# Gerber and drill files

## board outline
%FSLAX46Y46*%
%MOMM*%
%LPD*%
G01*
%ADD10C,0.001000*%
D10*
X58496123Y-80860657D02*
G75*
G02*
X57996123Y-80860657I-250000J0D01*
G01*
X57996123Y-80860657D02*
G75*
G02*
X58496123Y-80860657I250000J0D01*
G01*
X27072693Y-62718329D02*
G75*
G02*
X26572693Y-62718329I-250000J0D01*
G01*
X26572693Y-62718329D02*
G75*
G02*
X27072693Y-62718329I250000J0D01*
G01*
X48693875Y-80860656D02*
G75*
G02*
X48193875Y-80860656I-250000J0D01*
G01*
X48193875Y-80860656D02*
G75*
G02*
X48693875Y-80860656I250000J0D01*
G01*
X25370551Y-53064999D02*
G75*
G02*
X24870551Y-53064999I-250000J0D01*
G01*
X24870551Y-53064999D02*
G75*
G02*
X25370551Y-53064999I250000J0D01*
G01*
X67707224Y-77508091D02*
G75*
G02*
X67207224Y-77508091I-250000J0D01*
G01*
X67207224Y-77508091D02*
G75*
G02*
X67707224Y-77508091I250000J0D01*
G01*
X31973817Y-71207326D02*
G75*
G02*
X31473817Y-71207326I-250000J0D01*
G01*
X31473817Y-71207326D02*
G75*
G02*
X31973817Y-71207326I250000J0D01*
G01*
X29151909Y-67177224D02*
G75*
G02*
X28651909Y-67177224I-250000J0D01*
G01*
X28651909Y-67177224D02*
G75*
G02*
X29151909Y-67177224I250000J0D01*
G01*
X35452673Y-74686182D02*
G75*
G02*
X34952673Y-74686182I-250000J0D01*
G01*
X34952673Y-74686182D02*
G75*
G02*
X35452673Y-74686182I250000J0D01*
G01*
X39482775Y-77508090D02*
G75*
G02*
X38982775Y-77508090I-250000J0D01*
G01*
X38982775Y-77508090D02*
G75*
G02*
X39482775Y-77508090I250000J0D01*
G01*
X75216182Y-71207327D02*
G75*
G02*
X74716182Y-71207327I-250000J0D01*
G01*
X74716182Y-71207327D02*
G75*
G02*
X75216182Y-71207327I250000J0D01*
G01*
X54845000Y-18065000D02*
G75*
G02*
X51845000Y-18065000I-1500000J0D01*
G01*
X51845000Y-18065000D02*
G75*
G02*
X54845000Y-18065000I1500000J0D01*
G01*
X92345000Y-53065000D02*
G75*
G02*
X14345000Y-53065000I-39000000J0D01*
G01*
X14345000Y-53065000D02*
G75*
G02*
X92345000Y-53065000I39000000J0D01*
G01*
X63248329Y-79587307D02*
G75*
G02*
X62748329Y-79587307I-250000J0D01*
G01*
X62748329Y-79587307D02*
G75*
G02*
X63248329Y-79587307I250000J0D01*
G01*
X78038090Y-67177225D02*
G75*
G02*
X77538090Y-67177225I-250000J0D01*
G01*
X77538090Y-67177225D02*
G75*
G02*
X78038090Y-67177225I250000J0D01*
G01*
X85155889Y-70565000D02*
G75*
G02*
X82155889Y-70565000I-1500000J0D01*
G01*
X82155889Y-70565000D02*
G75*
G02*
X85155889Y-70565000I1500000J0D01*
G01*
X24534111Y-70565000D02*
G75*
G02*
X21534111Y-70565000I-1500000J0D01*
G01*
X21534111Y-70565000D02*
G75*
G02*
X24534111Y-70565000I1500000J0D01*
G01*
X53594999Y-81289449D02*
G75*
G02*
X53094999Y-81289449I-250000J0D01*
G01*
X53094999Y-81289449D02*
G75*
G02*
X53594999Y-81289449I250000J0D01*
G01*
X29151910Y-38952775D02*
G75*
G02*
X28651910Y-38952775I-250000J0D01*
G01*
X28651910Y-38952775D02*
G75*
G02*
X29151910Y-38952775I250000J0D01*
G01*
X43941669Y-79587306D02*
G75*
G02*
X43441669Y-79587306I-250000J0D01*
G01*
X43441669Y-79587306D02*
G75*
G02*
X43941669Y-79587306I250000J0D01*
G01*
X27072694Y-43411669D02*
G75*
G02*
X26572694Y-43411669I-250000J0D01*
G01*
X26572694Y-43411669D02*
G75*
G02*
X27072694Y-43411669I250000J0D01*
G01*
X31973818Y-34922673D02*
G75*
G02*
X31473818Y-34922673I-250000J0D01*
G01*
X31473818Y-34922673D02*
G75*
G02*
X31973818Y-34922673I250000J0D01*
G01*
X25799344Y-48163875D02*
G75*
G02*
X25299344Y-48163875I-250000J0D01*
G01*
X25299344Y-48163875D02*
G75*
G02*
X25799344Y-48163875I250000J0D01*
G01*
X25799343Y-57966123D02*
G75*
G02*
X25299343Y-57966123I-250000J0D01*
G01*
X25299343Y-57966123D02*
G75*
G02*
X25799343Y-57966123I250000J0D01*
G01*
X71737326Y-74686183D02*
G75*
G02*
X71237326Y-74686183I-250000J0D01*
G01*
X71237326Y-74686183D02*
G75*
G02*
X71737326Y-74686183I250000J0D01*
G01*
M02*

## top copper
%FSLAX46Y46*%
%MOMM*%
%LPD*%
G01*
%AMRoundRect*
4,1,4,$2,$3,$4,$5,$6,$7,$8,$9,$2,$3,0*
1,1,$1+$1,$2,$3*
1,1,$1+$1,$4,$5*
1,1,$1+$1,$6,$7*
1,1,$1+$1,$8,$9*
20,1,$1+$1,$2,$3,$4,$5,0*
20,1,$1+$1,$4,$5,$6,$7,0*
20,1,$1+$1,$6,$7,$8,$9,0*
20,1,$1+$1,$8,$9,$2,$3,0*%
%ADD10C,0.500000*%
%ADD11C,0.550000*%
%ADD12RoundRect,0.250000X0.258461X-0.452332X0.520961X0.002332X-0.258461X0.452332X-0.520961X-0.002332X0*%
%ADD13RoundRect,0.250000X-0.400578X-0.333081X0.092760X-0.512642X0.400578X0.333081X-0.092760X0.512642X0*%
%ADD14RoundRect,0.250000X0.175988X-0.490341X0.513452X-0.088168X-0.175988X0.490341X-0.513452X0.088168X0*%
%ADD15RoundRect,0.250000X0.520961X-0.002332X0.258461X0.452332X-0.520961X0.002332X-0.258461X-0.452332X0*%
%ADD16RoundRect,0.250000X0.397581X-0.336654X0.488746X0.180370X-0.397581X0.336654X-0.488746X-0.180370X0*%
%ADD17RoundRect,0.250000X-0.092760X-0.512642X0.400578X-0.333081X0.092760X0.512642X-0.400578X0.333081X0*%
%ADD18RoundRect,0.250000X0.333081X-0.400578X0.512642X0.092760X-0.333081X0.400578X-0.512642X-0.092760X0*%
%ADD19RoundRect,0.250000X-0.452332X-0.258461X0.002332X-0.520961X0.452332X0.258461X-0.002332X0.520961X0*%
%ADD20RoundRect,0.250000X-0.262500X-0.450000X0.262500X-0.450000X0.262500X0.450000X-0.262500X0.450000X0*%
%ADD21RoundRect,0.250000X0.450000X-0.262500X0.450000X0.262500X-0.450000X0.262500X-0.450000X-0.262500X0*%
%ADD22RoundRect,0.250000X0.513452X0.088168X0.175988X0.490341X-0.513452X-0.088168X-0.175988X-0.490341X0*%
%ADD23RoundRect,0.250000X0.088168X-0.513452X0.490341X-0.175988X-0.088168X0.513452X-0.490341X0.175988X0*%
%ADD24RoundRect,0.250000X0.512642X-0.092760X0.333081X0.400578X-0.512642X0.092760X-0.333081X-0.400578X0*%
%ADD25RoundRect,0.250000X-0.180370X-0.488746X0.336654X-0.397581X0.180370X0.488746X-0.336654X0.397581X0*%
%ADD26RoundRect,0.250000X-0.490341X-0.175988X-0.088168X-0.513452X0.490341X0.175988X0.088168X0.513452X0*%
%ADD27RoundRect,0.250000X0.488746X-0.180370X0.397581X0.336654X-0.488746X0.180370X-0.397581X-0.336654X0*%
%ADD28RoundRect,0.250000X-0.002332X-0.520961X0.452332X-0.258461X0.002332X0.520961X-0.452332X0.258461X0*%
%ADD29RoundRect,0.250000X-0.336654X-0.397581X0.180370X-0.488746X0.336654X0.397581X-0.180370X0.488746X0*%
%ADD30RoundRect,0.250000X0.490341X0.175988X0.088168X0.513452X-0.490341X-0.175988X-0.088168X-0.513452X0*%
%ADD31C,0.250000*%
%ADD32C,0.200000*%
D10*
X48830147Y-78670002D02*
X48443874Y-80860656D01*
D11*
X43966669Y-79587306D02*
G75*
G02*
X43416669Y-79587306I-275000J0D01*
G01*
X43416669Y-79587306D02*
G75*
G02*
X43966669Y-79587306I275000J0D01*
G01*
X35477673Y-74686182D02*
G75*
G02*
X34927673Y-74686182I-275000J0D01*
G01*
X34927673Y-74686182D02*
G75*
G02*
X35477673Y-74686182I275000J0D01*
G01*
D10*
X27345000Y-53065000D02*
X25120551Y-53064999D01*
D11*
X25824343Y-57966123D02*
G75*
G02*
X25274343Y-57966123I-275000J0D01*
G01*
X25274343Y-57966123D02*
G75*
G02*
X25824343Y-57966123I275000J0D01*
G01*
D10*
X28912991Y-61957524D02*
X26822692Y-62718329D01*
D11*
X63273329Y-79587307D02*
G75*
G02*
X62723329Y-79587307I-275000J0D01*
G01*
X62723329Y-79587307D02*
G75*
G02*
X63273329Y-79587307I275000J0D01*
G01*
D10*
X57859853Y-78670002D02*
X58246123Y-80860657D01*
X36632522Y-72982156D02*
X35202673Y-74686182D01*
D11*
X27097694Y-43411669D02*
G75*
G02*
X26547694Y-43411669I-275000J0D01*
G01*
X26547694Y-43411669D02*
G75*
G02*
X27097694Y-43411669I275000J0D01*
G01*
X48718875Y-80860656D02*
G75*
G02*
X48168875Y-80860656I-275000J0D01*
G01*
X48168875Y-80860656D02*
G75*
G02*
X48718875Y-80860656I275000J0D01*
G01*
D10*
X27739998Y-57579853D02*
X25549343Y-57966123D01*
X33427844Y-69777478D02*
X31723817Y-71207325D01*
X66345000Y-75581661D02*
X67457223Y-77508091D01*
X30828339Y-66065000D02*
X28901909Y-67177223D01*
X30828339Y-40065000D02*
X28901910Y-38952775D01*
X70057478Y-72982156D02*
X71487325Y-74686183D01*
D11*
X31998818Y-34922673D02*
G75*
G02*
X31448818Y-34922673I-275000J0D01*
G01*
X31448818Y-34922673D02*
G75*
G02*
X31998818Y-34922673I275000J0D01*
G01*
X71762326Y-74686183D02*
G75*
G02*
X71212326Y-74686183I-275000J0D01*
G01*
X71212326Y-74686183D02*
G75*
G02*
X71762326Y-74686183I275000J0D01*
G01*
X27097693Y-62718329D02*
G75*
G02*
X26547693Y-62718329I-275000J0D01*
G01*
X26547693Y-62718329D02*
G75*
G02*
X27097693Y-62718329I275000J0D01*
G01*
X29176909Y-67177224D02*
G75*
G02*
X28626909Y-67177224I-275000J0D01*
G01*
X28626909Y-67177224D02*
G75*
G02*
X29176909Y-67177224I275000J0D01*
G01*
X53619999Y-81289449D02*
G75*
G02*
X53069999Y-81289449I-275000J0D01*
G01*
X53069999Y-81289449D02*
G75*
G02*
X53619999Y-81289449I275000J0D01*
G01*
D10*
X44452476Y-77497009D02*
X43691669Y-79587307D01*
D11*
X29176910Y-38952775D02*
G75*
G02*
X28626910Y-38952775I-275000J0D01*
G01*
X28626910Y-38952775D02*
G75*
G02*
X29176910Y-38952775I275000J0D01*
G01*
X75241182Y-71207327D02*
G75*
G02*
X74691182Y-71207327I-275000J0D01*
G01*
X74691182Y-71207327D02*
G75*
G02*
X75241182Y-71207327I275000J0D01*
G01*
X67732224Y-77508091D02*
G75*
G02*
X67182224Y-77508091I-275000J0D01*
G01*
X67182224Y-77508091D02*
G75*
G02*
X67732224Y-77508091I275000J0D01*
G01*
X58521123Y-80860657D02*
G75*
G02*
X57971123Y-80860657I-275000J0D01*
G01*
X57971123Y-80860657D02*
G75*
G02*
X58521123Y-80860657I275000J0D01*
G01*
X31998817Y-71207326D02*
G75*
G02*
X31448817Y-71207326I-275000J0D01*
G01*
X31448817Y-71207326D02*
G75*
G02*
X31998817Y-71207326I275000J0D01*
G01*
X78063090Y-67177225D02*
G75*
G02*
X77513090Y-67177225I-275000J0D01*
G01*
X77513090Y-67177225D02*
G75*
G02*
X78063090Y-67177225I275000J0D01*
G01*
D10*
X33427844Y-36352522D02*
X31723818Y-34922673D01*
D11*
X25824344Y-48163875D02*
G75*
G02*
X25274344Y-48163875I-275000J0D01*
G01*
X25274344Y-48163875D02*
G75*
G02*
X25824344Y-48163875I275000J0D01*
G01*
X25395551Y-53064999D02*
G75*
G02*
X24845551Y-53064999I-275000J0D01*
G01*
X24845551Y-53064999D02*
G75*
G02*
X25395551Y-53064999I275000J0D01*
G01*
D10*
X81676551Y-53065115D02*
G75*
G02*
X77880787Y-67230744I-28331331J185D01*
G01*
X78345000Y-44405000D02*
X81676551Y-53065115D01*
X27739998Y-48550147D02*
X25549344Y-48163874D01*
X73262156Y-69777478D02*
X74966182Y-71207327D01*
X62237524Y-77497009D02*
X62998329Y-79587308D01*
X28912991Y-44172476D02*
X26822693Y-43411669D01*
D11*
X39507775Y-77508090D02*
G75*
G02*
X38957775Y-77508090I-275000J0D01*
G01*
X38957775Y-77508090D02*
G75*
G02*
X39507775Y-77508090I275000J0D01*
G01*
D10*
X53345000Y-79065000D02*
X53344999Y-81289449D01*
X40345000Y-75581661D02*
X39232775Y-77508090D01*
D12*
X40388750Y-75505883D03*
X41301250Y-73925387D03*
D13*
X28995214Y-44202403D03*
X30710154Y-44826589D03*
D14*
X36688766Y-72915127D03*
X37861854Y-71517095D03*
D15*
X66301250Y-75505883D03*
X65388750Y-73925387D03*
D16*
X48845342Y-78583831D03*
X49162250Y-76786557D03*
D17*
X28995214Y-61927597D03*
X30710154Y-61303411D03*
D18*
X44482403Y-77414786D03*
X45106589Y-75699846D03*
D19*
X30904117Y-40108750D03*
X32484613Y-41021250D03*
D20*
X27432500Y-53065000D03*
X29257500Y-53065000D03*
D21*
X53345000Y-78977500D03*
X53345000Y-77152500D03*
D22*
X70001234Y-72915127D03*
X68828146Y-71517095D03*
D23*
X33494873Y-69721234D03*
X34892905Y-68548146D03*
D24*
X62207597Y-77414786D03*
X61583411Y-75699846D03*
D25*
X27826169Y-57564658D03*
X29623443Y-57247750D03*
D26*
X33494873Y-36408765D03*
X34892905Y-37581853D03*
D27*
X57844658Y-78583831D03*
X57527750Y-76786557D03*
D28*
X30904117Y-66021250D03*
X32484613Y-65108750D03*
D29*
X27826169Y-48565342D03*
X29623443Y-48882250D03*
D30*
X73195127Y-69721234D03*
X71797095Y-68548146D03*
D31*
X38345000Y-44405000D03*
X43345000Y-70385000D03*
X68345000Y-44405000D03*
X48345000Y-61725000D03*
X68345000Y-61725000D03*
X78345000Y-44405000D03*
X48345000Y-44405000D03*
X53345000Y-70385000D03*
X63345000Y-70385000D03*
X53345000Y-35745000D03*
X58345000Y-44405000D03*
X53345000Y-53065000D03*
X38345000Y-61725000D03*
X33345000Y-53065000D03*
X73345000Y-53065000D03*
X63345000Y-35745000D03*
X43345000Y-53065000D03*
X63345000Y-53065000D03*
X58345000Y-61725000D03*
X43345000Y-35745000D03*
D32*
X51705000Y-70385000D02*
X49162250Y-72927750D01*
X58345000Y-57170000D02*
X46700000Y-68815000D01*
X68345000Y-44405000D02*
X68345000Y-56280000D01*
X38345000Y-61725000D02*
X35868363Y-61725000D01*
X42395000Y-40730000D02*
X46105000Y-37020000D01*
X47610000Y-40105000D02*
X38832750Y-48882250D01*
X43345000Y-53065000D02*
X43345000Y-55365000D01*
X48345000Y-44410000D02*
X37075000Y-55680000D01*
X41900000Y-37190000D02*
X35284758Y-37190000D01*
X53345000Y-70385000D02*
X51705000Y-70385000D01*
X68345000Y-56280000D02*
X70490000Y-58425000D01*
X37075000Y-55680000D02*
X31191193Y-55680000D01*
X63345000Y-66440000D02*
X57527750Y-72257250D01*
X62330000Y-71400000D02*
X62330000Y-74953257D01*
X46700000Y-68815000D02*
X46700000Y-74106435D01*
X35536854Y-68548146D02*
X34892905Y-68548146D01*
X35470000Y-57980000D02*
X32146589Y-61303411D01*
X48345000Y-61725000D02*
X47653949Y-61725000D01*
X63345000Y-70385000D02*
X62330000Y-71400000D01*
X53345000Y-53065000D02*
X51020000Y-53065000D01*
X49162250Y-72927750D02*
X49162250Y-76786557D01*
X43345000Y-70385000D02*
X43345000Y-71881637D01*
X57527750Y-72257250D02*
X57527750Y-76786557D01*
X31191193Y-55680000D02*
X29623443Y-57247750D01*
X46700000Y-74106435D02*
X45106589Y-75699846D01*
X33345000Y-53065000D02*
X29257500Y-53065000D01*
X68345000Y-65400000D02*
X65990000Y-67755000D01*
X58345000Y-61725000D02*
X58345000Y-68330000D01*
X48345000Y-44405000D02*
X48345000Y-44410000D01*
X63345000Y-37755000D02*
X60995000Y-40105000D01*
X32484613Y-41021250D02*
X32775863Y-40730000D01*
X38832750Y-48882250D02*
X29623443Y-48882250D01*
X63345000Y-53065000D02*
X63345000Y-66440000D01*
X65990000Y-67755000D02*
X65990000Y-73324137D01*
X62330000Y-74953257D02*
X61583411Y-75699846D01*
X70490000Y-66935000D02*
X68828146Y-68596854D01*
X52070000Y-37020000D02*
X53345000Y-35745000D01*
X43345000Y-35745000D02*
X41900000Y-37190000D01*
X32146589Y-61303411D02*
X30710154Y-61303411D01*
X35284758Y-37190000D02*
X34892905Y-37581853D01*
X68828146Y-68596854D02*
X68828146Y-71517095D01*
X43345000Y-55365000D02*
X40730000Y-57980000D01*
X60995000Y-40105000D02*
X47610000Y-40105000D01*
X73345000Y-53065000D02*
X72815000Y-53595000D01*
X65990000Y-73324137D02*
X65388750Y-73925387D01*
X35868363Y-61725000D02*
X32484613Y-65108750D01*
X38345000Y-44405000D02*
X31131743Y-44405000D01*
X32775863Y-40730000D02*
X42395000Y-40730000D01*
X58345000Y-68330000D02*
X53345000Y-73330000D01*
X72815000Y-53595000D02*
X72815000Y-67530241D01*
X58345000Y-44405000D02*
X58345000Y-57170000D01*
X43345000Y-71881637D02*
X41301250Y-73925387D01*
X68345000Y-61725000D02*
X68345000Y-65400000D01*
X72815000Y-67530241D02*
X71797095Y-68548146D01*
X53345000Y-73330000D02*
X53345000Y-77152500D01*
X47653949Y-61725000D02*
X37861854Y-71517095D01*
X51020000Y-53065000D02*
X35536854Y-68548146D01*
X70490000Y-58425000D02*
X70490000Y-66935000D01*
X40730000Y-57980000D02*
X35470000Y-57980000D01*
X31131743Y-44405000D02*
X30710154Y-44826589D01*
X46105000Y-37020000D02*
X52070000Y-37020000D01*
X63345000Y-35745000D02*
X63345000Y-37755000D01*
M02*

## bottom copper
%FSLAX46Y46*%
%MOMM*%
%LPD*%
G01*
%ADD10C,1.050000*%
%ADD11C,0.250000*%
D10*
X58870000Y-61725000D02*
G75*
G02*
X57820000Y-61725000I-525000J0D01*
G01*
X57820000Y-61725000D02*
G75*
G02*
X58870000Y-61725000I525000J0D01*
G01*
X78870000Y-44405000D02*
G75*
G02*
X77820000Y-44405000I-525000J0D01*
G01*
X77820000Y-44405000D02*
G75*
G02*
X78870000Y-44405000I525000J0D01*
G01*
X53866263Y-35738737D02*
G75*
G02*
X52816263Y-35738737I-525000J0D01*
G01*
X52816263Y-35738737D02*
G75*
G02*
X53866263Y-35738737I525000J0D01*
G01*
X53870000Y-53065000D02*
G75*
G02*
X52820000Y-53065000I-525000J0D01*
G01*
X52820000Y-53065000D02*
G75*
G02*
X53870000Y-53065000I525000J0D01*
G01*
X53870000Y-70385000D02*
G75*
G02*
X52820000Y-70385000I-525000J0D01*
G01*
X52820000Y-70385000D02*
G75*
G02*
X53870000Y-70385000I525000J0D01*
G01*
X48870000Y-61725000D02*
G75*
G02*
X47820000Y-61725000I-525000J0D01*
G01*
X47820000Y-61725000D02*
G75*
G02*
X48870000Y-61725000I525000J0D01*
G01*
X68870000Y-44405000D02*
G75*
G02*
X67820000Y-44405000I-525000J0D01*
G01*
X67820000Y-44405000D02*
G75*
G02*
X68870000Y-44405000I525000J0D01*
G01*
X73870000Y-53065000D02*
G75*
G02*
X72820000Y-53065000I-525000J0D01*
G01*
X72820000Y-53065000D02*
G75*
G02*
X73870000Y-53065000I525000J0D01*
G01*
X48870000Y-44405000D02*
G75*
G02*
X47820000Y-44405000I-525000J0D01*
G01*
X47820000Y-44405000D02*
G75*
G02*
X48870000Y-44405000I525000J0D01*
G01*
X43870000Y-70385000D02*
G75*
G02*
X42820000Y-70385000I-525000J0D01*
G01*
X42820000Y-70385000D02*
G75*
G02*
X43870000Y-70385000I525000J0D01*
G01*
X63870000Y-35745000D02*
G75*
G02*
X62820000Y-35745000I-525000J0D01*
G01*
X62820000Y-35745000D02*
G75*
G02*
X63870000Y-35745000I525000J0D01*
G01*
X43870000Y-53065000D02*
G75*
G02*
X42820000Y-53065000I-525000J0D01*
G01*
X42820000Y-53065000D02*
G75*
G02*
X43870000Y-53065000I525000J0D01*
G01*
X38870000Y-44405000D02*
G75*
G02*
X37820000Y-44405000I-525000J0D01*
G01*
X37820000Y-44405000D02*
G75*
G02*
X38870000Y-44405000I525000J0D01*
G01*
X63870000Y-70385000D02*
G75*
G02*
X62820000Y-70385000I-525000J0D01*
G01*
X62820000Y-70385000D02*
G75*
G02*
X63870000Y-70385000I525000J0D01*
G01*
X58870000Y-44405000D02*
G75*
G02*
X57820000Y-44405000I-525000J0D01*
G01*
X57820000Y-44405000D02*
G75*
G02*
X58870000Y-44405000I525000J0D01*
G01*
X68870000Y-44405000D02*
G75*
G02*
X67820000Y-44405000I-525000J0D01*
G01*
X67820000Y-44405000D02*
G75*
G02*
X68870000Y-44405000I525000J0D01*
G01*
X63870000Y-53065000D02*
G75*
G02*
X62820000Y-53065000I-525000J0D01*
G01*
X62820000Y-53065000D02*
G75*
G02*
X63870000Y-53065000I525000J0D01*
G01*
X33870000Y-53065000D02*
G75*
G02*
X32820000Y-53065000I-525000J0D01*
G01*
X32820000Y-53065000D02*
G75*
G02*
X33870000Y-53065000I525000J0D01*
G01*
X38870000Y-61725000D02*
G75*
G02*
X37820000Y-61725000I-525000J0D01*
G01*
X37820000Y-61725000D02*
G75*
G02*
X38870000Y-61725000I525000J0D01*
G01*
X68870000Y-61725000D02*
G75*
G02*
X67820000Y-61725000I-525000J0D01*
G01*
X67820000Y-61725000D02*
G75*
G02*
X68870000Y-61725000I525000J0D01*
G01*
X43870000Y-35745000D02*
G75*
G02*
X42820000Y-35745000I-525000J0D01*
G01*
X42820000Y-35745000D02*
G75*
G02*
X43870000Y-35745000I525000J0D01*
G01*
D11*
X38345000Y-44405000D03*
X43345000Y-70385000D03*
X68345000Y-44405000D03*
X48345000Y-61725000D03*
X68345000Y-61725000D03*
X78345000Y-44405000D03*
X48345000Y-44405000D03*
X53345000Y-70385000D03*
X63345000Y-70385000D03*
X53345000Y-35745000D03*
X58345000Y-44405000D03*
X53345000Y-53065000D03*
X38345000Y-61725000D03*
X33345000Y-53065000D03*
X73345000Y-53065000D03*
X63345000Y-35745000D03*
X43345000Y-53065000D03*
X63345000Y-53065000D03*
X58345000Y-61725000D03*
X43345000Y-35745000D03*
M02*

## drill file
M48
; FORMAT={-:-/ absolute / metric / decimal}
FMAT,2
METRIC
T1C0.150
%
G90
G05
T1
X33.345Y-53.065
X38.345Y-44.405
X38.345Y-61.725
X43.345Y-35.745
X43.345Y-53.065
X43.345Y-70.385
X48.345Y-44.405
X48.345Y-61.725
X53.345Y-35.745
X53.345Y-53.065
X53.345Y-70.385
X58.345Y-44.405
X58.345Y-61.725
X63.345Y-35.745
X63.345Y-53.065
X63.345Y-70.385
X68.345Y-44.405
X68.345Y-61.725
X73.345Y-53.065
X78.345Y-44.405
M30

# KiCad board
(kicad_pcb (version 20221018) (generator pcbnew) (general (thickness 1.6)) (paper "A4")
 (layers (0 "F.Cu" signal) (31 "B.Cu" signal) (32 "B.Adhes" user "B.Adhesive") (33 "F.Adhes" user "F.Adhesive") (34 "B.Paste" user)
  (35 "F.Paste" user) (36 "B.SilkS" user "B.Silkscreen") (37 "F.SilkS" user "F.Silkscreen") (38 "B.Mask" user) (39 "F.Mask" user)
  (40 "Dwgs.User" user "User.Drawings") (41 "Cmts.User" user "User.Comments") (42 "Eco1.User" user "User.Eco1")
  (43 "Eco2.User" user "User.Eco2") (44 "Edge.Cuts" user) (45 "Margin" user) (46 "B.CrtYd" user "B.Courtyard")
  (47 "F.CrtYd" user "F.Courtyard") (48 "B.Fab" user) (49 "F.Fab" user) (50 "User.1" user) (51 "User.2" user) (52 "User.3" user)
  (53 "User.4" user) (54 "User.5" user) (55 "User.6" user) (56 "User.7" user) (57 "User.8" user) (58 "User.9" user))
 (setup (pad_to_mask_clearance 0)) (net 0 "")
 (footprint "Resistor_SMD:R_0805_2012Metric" (layer "F.Cu") (at 40.845 74.715635 60)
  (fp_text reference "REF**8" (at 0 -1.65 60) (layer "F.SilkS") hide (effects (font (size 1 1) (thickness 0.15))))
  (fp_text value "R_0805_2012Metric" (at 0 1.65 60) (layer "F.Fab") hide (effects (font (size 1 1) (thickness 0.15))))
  (pad "1" smd roundrect (at -0.9125 0 60) (size 1.025 1.4) (layers "F.Cu" "F.Paste" "F.Mask") (roundrect_rratio 0.243902))
  (pad "2" smd roundrect (at 0.9125 0 60) (size 1.025 1.4) (layers "F.Cu" "F.Paste" "F.Mask") (roundrect_rratio 0.243902)))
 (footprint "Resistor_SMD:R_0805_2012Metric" (layer "F.Cu") (at 29.852684 44.514496 -20)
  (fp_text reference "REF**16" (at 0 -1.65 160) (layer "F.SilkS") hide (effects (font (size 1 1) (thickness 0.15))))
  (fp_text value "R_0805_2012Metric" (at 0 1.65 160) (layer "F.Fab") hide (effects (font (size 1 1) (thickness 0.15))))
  (pad "1" smd roundrect (at -0.9125 0 340) (size 1.025 1.4) (layers "F.Cu" "F.Paste" "F.Mask") (roundrect_rratio 0.243902))
  (pad "2" smd roundrect (at 0.9125 0 340) (size 1.025 1.4) (layers "F.Cu" "F.Paste" "F.Mask") (roundrect_rratio 0.243902)))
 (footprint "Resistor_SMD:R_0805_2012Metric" (layer "F.Cu") (at 37.27531 72.216111 50)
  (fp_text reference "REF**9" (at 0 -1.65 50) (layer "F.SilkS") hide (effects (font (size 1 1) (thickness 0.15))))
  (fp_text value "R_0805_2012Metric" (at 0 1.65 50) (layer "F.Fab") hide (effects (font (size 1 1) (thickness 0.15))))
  (pad "1" smd roundrect (at -0.9125 0 50) (size 1.025 1.4) (layers "F.Cu" "F.Paste" "F.Mask") (roundrect_rratio 0.243902))
  (pad "2" smd roundrect (at 0.9125 0 50) (size 1.025 1.4) (layers "F.Cu" "F.Paste" "F.Mask") (roundrect_rratio 0.243902)))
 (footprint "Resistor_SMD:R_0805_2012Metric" (layer "F.Cu") (at 65.845 74.715635 120)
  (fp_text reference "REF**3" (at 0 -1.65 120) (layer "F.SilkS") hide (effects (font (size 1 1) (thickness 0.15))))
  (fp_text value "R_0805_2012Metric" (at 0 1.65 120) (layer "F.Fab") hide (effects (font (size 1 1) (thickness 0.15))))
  (pad "1" smd roundrect (at -0.9125 0 120) (size 1.025 1.4) (layers "F.Cu" "F.Paste" "F.Mask") (roundrect_rratio 0.243902))
  (pad "2" smd roundrect (at 0.9125 0 120) (size 1.025 1.4) (layers "F.Cu" "F.Paste" "F.Mask") (roundrect_rratio 0.243902)))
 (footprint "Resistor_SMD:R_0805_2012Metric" (layer "F.Cu") (at 49.003796 77.685194 80)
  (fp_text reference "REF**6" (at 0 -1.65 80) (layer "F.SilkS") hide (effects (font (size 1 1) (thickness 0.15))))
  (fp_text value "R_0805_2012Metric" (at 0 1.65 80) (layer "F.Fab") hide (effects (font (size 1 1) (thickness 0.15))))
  (pad "1" smd roundrect (at -0.9125 0 80) (size 1.025 1.4) (layers "F.Cu" "F.Paste" "F.Mask") (roundrect_rratio 0.243902))
  (pad "2" smd roundrect (at 0.9125 0 80) (size 1.025 1.4) (layers "F.Cu" "F.Paste" "F.Mask") (roundrect_rratio 0.243902)))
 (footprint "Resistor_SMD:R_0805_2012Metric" (layer "F.Cu") (at 29.852684 61.615504 20)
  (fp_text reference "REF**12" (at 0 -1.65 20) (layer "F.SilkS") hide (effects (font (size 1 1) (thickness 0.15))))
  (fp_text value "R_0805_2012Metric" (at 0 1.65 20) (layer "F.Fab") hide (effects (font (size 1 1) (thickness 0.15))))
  (pad "1" smd roundrect (at -0.9125 0 20) (size 1.025 1.4) (layers "F.Cu" "F.Paste" "F.Mask") (roundrect_rratio 0.243902))
  (pad "2" smd roundrect (at 0.9125 0 20) (size 1.025 1.4) (layers "F.Cu" "F.Paste" "F.Mask") (roundrect_rratio 0.243902)))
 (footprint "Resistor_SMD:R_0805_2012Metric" (layer "F.Cu") (at 44.794496 76.557316 70)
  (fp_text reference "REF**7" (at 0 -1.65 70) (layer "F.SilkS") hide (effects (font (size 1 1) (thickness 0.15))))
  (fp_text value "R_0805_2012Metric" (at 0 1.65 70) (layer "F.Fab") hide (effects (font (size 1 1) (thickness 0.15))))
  (pad "1" smd roundrect (at -0.9125 0 70) (size 1.025 1.4) (layers "F.Cu" "F.Paste" "F.Mask") (roundrect_rratio 0.243902))
  (pad "2" smd roundrect (at 0.9125 0 70) (size 1.025 1.4) (layers "F.Cu" "F.Paste" "F.Mask") (roundrect_rratio 0.243902)))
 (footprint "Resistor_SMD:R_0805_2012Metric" (layer "F.Cu") (at 31.694365 40.565 -30)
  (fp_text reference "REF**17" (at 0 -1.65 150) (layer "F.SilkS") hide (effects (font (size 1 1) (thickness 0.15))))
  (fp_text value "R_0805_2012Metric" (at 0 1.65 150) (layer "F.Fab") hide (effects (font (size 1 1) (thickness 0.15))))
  (pad "1" smd roundrect (at -0.9125 0 330) (size 1.025 1.4) (layers "F.Cu" "F.Paste" "F.Mask") (roundrect_rratio 0.243902))
  (pad "2" smd roundrect (at 0.9125 0 330) (size 1.025 1.4) (layers "F.Cu" "F.Paste" "F.Mask") (roundrect_rratio 0.243902)))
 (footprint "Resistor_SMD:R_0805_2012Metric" (layer "F.Cu") (at 28.345 53.065)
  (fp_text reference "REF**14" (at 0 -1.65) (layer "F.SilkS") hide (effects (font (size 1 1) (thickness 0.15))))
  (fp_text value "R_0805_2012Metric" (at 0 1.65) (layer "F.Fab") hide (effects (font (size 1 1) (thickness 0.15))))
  (pad "1" smd roundrect (at -0.9125 0) (size 1.025 1.4) (layers "F.Cu" "F.Paste" "F.Mask") (roundrect_rratio 0.243902))
  (pad "2" smd roundrect (at 0.9125 0) (size 1.025 1.4) (layers "F.Cu" "F.Paste" "F.Mask") (roundrect_rratio 0.243902)))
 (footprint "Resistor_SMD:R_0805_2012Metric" (layer "F.Cu") (at 53.345 78.065 90)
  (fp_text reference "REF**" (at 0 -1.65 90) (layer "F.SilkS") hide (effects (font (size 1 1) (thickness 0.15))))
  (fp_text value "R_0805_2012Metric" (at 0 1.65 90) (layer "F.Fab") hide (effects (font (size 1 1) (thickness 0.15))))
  (pad "1" smd roundrect (at -0.9125 0 90) (size 1.025 1.4) (layers "F.Cu" "F.Paste" "F.Mask") (roundrect_rratio 0.243902))
  (pad "2" smd roundrect (at 0.9125 0 90) (size 1.025 1.4) (layers "F.Cu" "F.Paste" "F.Mask") (roundrect_rratio 0.243902)))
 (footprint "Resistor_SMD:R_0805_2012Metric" (layer "F.Cu") (at 69.41469 72.216111 130)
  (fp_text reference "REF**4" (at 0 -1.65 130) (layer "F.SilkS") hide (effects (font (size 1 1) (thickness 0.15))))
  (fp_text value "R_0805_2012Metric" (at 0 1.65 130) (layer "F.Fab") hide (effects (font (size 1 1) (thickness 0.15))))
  (pad "1" smd roundrect (at -0.9125 0 130) (size 1.025 1.4) (layers "F.Cu" "F.Paste" "F.Mask") (roundrect_rratio 0.243902))
  (pad "2" smd roundrect (at 0.9125 0 130) (size 1.025 1.4) (layers "F.Cu" "F.Paste" "F.Mask") (roundrect_rratio 0.243902)))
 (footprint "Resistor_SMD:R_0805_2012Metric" (layer "F.Cu") (at 34.193889 69.13469 40)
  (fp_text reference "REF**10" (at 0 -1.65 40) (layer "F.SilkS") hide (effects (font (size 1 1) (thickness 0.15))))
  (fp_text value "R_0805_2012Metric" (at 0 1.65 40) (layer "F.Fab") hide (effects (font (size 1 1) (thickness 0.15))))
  (pad "1" smd roundrect (at -0.9125 0 40) (size 1.025 1.4) (layers "F.Cu" "F.Paste" "F.Mask") (roundrect_rratio 0.243902))
  (pad "2" smd roundrect (at 0.9125 0 40) (size 1.025 1.4) (layers "F.Cu" "F.Paste" "F.Mask") (roundrect_rratio 0.243902)))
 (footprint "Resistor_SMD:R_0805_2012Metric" (layer "F.Cu") (at 61.895504 76.557316 110)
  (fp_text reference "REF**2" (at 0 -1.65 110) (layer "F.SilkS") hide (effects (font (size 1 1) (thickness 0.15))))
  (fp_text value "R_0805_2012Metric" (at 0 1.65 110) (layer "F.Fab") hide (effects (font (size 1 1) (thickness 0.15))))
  (pad "1" smd roundrect (at -0.9125 0 110) (size 1.025 1.4) (layers "F.Cu" "F.Paste" "F.Mask") (roundrect_rratio 0.243902))
  (pad "2" smd roundrect (at 0.9125 0 110) (size 1.025 1.4) (layers "F.Cu" "F.Paste" "F.Mask") (roundrect_rratio 0.243902)))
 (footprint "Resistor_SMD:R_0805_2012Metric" (layer "F.Cu") (at 28.724806 57.406204 10)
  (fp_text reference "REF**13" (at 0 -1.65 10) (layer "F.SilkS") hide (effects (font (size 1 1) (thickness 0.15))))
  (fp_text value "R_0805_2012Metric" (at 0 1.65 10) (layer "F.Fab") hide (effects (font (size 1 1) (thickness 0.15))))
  (pad "1" smd roundrect (at -0.9125 0 10) (size 1.025 1.4) (layers "F.Cu" "F.Paste" "F.Mask") (roundrect_rratio 0.243902))
  (pad "2" smd roundrect (at 0.9125 0 10) (size 1.025 1.4) (layers "F.Cu" "F.Paste" "F.Mask") (roundrect_rratio 0.243902)))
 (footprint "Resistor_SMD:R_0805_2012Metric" (layer "F.Cu") (at 34.193889 36.995309 -40)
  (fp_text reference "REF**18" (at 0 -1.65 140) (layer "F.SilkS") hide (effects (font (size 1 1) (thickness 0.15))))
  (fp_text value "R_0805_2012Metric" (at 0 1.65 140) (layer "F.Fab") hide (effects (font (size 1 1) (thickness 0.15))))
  (pad "1" smd roundrect (at -0.9125 0 320) (size 1.025 1.4) (layers "F.Cu" "F.Paste" "F.Mask") (roundrect_rratio 0.243902))
  (pad "2" smd roundrect (at 0.9125 0 320) (size 1.025 1.4) (layers "F.Cu" "F.Paste" "F.Mask") (roundrect_rratio 0.243902)))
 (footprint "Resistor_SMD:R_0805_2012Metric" (layer "F.Cu") (at 57.686204 77.685194 100)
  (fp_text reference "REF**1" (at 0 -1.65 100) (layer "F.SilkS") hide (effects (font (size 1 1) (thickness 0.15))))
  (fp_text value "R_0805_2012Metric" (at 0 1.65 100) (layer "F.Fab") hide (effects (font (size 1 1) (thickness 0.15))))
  (pad "1" smd roundrect (at -0.9125 0 100) (size 1.025 1.4) (layers "F.Cu" "F.Paste" "F.Mask") (roundrect_rratio 0.243902))
  (pad "2" smd roundrect (at 0.9125 0 100) (size 1.025 1.4) (layers "F.Cu" "F.Paste" "F.Mask") (roundrect_rratio 0.243902)))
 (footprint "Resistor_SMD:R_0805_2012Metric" (layer "F.Cu") (at 31.694365 65.565 30)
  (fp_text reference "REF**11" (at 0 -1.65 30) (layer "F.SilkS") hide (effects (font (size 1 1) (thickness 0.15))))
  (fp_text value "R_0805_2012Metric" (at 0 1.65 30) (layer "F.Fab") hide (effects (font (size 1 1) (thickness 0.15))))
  (pad "1" smd roundrect (at -0.9125 0 30) (size 1.025 1.4) (layers "F.Cu" "F.Paste" "F.Mask") (roundrect_rratio 0.243902))
  (pad "2" smd roundrect (at 0.9125 0 30) (size 1.025 1.4) (layers "F.Cu" "F.Paste" "F.Mask") (roundrect_rratio 0.243902)))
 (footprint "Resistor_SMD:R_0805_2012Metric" (layer "F.Cu") (at 28.724806 48.723796 -10)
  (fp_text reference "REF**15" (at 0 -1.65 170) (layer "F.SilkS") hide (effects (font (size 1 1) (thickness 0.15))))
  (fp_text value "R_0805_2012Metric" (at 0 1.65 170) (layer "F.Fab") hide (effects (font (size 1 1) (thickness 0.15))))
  (pad "1" smd roundrect (at -0.9125 0 350) (size 1.025 1.4) (layers "F.Cu" "F.Paste" "F.Mask") (roundrect_rratio 0.243902))
  (pad "2" smd roundrect (at 0.9125 0 350) (size 1.025 1.4) (layers "F.Cu" "F.Paste" "F.Mask") (roundrect_rratio 0.243902)))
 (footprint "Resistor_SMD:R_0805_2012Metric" (layer "F.Cu") (at 72.496111 69.13469 140)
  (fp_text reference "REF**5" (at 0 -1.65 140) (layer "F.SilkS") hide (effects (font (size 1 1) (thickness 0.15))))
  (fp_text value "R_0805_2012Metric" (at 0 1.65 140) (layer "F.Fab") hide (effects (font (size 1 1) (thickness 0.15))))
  (pad "1" smd roundrect (at -0.9125 0 140) (size 1.025 1.4) (layers "F.Cu" "F.Paste" "F.Mask") (roundrect_rratio 0.243902))
  (pad "2" smd roundrect (at 0.9125 0 140) (size 1.025 1.4) (layers "F.Cu" "F.Paste" "F.Mask") (roundrect_rratio 0.243902)))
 (gr_line (start 48.830147 78.670002) (end 48.443874 80.860656) (stroke (width 0.5) (type solid)) (layer "F.Cu"))
 (gr_circle (center 43.691669 79.587306) (end 44.161515 79.416296) (stroke (width 0.1) (type solid)) (fill solid) (layer "F.Cu"))
 (gr_circle (center 35.202673 74.686182) (end 35.702673 74.686182) (stroke (width 0.1) (type solid)) (fill solid) (layer "F.Cu"))
 (gr_line (start 27.345 53.065) (end 25.120551 53.064999) (stroke (width 0.5) (type solid)) (layer "F.Cu"))
 (gr_circle (center 25.549343 57.966123) (end 25.932365 58.287517) (stroke (width 0.1) (type solid)) (fill solid) (layer "F.Cu"))
 (gr_line (start 28.912991 61.957524) (end 26.822692 62.718329) (stroke (width 0.5) (type solid)) (layer "F.Cu"))
 (gr_circle (center 62.998329 79.587307) (end 63.248329 79.154294) (stroke (width 0.1) (type solid)) (fill solid) (layer "F.Cu"))
 (gr_line (start 57.859853 78.670002) (end 58.246123 80.860657) (stroke (width 0.5) (type solid)) (layer "F.Cu"))
 (gr_line (start 36.632522 72.982156) (end 35.202673 74.686182) (stroke (width 0.5) (type solid)) (layer "F.Cu"))
 (gr_circle (center 26.822694 43.411669) (end 26.993704 43.881515) (stroke (width 0.1) (type solid)) (fill solid) (layer "F.Cu"))
 (gr_circle (center 48.443875 80.860656) (end 48.876888 80.610656) (stroke (width 0.1) (type solid)) (fill solid) (layer "F.Cu"))
 (gr_line (start 27.739998 57.579853) (end 25.549343 57.966123) (stroke (width 0.5) (type solid)) (layer "F.Cu"))
 (gr_line (start 33.427844 69.777478) (end 31.723817 71.207325) (stroke (width 0.5) (type solid)) (layer "F.Cu"))
 (gr_line (start 66.345 75.581661) (end 67.457223 77.508091) (stroke (width 0.5) (type solid)) (layer "F.Cu"))
 (gr_line (start 30.828339 66.065) (end 28.901909 67.177223) (stroke (width 0.5) (type solid)) (layer "F.Cu"))
 (gr_line (start 30.828339 40.065) (end 28.90191 38.952775) (stroke (width 0.5) (type solid)) (layer "F.Cu"))
 (gr_line (start 70.057478 72.982156) (end 71.487325 74.686183) (stroke (width 0.5) (type solid)) (layer "F.Cu"))
 (gr_circle (center 31.723818 34.922673) (end 31.723818 35.422673) (stroke (width 0.1) (type solid)) (fill solid) (layer "F.Cu"))
 (gr_circle (center 71.487326 74.686183) (end 71.57415 74.193779) (stroke (width 0.1) (type solid)) (fill solid) (layer "F.Cu"))
 (gr_circle (center 26.822693 62.718329) (end 27.255706 62.968329) (stroke (width 0.1) (type solid)) (fill solid) (layer "F.Cu"))
 (gr_circle (center 28.901909 67.177224) (end 29.371755 67.348234) (stroke (width 0.1) (type solid)) (fill solid) (layer "F.Cu"))
 (gr_circle (center 53.344999 81.289449) (end 53.728021 80.968055) (stroke (width 0.1) (type solid)) (fill solid) (layer "F.Cu"))
 (gr_line (start 44.452476 77.497009) (end 43.691669 79.587307) (stroke (width 0.5) (type solid)) (layer "F.Cu"))
 (gr_circle (center 28.90191 38.952775) (end 28.988734 39.445179) (stroke (width 0.1) (type solid)) (fill solid) (layer "F.Cu"))
 (gr_circle (center 74.966182 71.207327) (end 74.966182 70.707327) (stroke (width 0.1) (type solid)) (fill solid) (layer "F.Cu"))
 (gr_circle (center 67.457224 77.508091) (end 67.628234 77.038245) (stroke (width 0.1) (type solid)) (fill solid) (layer "F.Cu"))
 (gr_circle (center 58.246123 80.860657) (end 58.567517 80.477635) (stroke (width 0.1) (type solid)) (fill solid) (layer "F.Cu"))
 (gr_circle (center 31.723817 71.207326) (end 32.216221 71.29415) (stroke (width 0.1) (type solid)) (fill solid) (layer "F.Cu"))
 (gr_circle (center 77.78809 67.177225) (end 77.701266 66.684821) (stroke (width 0.1) (type solid)) (fill solid) (layer "F.Cu"))
 (gr_line (start 33.427844 36.352522) (end 31.723818 34.922673) (stroke (width 0.5) (type solid)) (layer "F.Cu"))
 (gr_circle (center 25.549344 48.163875) (end 25.799344 48.596888) (stroke (width 0.1) (type solid)) (fill solid) (layer "F.Cu"))
 (gr_circle (center 25.120551 53.064999) (end 25.441945 53.448021) (stroke (width 0.1) (type solid)) (fill solid) (layer "F.Cu"))
 (gr_arc (start 81.676551 53.065115) (mid 80.711139 60.397791) (end 77.880788 67.230745) (stroke (width 0.5) (type default)) (layer "F.Cu"))
 (gr_line (start 78.345 44.405) (end 81.676551 53.065115) (stroke (width 0.5) (type solid)) (layer "F.Cu"))
 (gr_line (start 27.739998 48.550147) (end 25.549344 48.163874) (stroke (width 0.5) (type solid)) (layer "F.Cu"))
 (gr_line (start 73.262156 69.777478) (end 74.966182 71.207327) (stroke (width 0.5) (type solid)) (layer "F.Cu"))
 (gr_line (start 62.237524 77.497009) (end 62.998329 79.587308) (stroke (width 0.5) (type solid)) (layer "F.Cu"))
 (gr_line (start 28.912991 44.172476) (end 26.822693 43.411669) (stroke (width 0.5) (type solid)) (layer "F.Cu"))
 (gr_circle (center 39.232775 77.50809) (end 39.725179 77.421266) (stroke (width 0.1) (type solid)) (fill solid) (layer "F.Cu"))
 (gr_line (start 53.345 79.065) (end 53.344999 81.289449) (stroke (width 0.5) (type solid)) (layer "F.Cu"))
 (gr_line (start 40.345 75.581661) (end 39.232775 77.50809) (stroke (width 0.5) (type solid)) (layer "F.Cu"))
 (gr_circle (center 58.345 61.725) (end 59.345 61.725) (stroke (width 0.1) (type solid)) (fill solid) (layer "B.Cu"))
 (gr_circle (center 78.345 44.405) (end 79.345 44.405) (stroke (width 0.1) (type solid)) (fill solid) (layer "B.Cu"))
 (gr_circle (center 53.341263 35.738737) (end 54.341263 35.738737) (stroke (width 0.1) (type solid)) (fill solid) (layer "B.Cu"))
 (gr_circle (center 53.345 53.065) (end 54.345 53.065) (stroke (width 0.1) (type solid)) (fill solid) (layer "B.Cu"))
 (gr_circle (center 53.345 70.385) (end 54.345 70.385) (stroke (width 0.1) (type solid)) (fill solid) (layer "B.Cu"))
 (gr_circle (center 48.345 61.725) (end 49.345 61.725) (stroke (width 0.1) (type solid)) (fill solid) (layer "B.Cu"))
 (gr_circle (center 68.345 44.405) (end 69.345 44.405) (stroke (width 0.1) (type solid)) (fill solid) (layer "B.Cu"))
 (gr_circle (center 73.345 53.065) (end 74.345 53.065) (stroke (width 0.1) (type solid)) (fill solid) (layer "B.Cu"))
 (gr_circle (center 48.345 44.405) (end 49.345 44.405) (stroke (width 0.1) (type solid)) (fill solid) (layer "B.Cu"))
 (gr_circle (center 43.345 70.385) (end 44.345 70.385) (stroke (width 0.1) (type solid)) (fill solid) (layer "B.Cu"))
 (gr_circle (center 63.345 35.745) (end 64.345 35.745) (stroke (width 0.1) (type solid)) (fill solid) (layer "B.Cu"))
 (gr_circle (center 43.345 53.065) (end 44.345 53.065) (stroke (width 0.1) (type solid)) (fill solid) (layer "B.Cu"))
 (gr_circle (center 38.345 44.405) (end 39.345 44.405) (stroke (width 0.1) (type solid)) (fill solid) (layer "B.Cu"))
 (gr_circle (center 63.345 70.385) (end 64.345 70.385) (stroke (width 0.1) (type solid)) (fill solid) (layer "B.Cu"))
 (gr_circle (center 58.345 44.405) (end 59.345 44.405) (stroke (width 0.1) (type solid)) (fill solid) (layer "B.Cu"))
 (gr_circle (center 68.345 44.405) (end 69.345 44.405) (stroke (width 0.1) (type solid)) (fill solid) (layer "B.Cu"))
 (gr_circle (center 63.345 53.065) (end 64.345 53.065) (stroke (width 0.1) (type solid)) (fill solid) (layer "B.Cu"))
 (gr_circle (center 33.345 53.065) (end 34.345 53.065) (stroke (width 0.1) (type solid)) (fill solid) (layer "B.Cu"))
 (gr_circle (center 38.345 61.725) (end 39.345 61.725) (stroke (width 0.1) (type solid)) (fill solid) (layer "B.Cu"))
 (gr_circle (center 68.345 61.725) (end 69.345 61.725) (stroke (width 0.1) (type solid)) (fill solid) (layer "B.Cu"))
 (gr_circle (center 43.345 35.745) (end 44.345 35.745) (stroke (width 0.1) (type solid)) (fill solid) (layer "B.Cu"))
 (gr_circle (center 58.246123 80.860657) (end 58.40682 80.669146) (stroke (width 0.001) (type solid)) (fill none) (layer "Edge.Cuts"))
 (gr_circle (center 26.822693 62.718329) (end 27.039199 62.843329) (stroke (width 0.001) (type solid)) (fill none) (layer "Edge.Cuts"))
 (gr_circle (center 48.443875 80.860656) (end 48.660381 80.735656) (stroke (width 0.001) (type solid)) (fill none) (layer "Edge.Cuts"))
 (gr_circle (center 25.120551 53.064999) (end 25.281248 53.25651) (stroke (width 0.001) (type solid)) (fill none) (layer "Edge.Cuts"))
 (gr_circle (center 67.457224 77.508091) (end 67.542729 77.273168) (stroke (width 0.001) (type solid)) (fill none) (layer "Edge.Cuts"))
 (gr_circle (center 31.723817 71.207326) (end 31.970019 71.250738) (stroke (width 0.001) (type solid)) (fill none) (layer "Edge.Cuts"))
 (gr_circle (center 28.901909 67.177224) (end 29.136832 67.262729) (stroke (width 0.001) (type solid)) (fill none) (layer "Edge.Cuts"))
 (gr_circle (center 35.202673 74.686182) (end 35.452673 74.686182) (stroke (width 0.001) (type solid)) (fill none) (layer "Edge.Cuts"))
 (gr_circle (center 39.232775 77.50809) (end 39.478977 77.464678) (stroke (width 0.001) (type solid)) (fill none) (layer "Edge.Cuts"))
 (gr_circle (center 74.966182 71.207327) (end 74.966182 70.957327) (stroke (width 0.001) (type solid)) (fill none) (layer "Edge.Cuts"))
 (gr_circle (center 53.345 18.065) (end 54.845 18.065) (stroke (width 0.001) (type default)) (fill none) (layer "Edge.Cuts"))
 (gr_circle (center 53.345 53.065) (end 92.345 53.065) (stroke (width 0.001) (type solid)) (fill none) (layer "Edge.Cuts"))
 (gr_circle (center 62.998329 79.587307) (end 63.123329 79.370801) (stroke (width 0.001) (type solid)) (fill none) (layer "Edge.Cuts"))
 (gr_circle (center 77.78809 67.177225) (end 77.744678 66.931023) (stroke (width 0.001) (type solid)) (fill none) (layer "Edge.Cuts"))
 (gr_circle (center 83.655889 70.565) (end 85.155889 70.565) (stroke (width 0.001) (type default)) (fill none) (layer "Edge.Cuts"))
 (gr_circle (center 23.034111 70.565) (end 24.534111 70.565) (stroke (width 0.001) (type default)) (fill none) (layer "Edge.Cuts"))
 (gr_circle (center 53.344999 81.289449) (end 53.53651 81.128752) (stroke (width 0.001) (type solid)) (fill none) (layer "Edge.Cuts"))
 (gr_circle (center 28.90191 38.952775) (end 28.945322 39.198977) (stroke (width 0.001) (type solid)) (fill none) (layer "Edge.Cuts"))
 (gr_circle (center 43.691669 79.587306) (end 43.926592 79.501801) (stroke (width 0.001) (type solid)) (fill none) (layer "Edge.Cuts"))
 (gr_circle (center 26.822694 43.411669) (end 26.908199 43.646592) (stroke (width 0.001) (type solid)) (fill none) (layer "Edge.Cuts"))
 (gr_circle (center 31.723818 34.922673) (end 31.723818 35.172673) (stroke (width 0.001) (type solid)) (fill none) (layer "Edge.Cuts"))
 (gr_circle (center 25.549344 48.163875) (end 25.674344 48.380381) (stroke (width 0.001) (type solid)) (fill none) (layer "Edge.Cuts"))
 (gr_circle (center 25.549343 57.966123) (end 25.740854 58.12682) (stroke (width 0.001) (type solid)) (fill none) (layer "Edge.Cuts"))
 (gr_circle (center 71.487326 74.686183) (end 71.530738 74.439981) (stroke (width 0.001) (type solid)) (fill none) (layer "Edge.Cuts"))
 (segment (start 51.705 70.385) (end 49.16225 72.92775) (width 0.2) (layer "F.Cu") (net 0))
 (segment (start 58.345 57.17) (end 46.7 68.815) (width 0.2) (layer "F.Cu") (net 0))
 (segment (start 68.345 44.405) (end 68.345 56.28) (width 0.2) (layer "F.Cu") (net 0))
 (segment (start 38.345 61.725) (end 35.868363 61.725) (width 0.2) (layer "F.Cu") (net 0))
 (segment (start 42.395 40.73) (end 46.105 37.02) (width 0.2) (layer "F.Cu") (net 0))
 (segment (start 47.61 40.105) (end 38.83275 48.88225) (width 0.2) (layer "F.Cu") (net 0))
 (segment (start 43.345 53.065) (end 43.345 55.365) (width 0.2) (layer "F.Cu") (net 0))
 (segment (start 48.345 44.41) (end 37.075 55.68) (width 0.2) (layer "F.Cu") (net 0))
 (segment (start 41.9 37.19) (end 35.284758 37.19) (width 0.2) (layer "F.Cu") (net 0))
 (segment (start 53.345 70.385) (end 51.705 70.385) (width 0.2) (layer "F.Cu") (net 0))
 (segment (start 68.345 56.28) (end 70.49 58.425) (width 0.2) (layer "F.Cu") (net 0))
 (segment (start 37.075 55.68) (end 31.191193 55.68) (width 0.2) (layer "F.Cu") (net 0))
 (segment (start 63.345 66.44) (end 57.52775 72.25725) (width 0.2) (layer "F.Cu") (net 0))
 (segment (start 62.33 71.4) (end 62.33 74.953257) (width 0.2) (layer "F.Cu") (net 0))
 (segment (start 46.7 68.815) (end 46.7 74.106435) (width 0.2) (layer "F.Cu") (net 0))
 (segment (start 35.536854 68.548146) (end 34.892905 68.548146) (width 0.2) (layer "F.Cu") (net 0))
 (segment (start 35.47 57.98) (end 32.146589 61.303411) (width 0.2) (layer "F.Cu") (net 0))
 (segment (start 48.345 61.725) (end 47.653949 61.725) (width 0.2) (layer "F.Cu") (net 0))
 (segment (start 63.345 70.385) (end 62.33 71.4) (width 0.2) (layer "F.Cu") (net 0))
 (segment (start 53.345 53.065) (end 51.02 53.065) (width 0.2) (layer "F.Cu") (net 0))
 (segment (start 49.16225 72.92775) (end 49.16225 76.786557) (width 0.2) (layer "F.Cu") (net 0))
 (segment (start 43.345 70.385) (end 43.345 71.881637) (width 0.2) (layer "F.Cu") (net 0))
 (segment (start 57.52775 72.25725) (end 57.52775 76.786557) (width 0.2) (layer "F.Cu") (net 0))
 (segment (start 31.191193 55.68) (end 29.623443 57.24775) (width 0.2) (layer "F.Cu") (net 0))
 (segment (start 46.7 74.106435) (end 45.106589 75.699846) (width 0.2) (layer "F.Cu") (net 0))
 (segment (start 33.345 53.065) (end 29.2575 53.065) (width 0.2) (layer "F.Cu") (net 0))
 (segment (start 68.345 65.4) (end 65.99 67.755) (width 0.2) (layer "F.Cu") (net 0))
 (segment (start 58.345 61.725) (end 58.345 68.33) (width 0.2) (layer "F.Cu") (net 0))
 (segment (start 48.345 44.405) (end 48.345 44.41) (width 0.2) (layer "F.Cu") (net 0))
 (segment (start 63.345 37.755) (end 60.995 40.105) (width 0.2) (layer "F.Cu") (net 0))
 (segment (start 32.484613 41.02125) (end 32.775863 40.73) (width 0.2) (layer "F.Cu") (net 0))
 (segment (start 38.83275 48.88225) (end 29.623443 48.88225) (width 0.2) (layer "F.Cu") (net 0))
 (segment (start 63.345 53.065) (end 63.345 66.44) (width 0.2) (layer "F.Cu") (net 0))
 (segment (start 65.99 67.755) (end 65.99 73.324137) (width 0.2) (layer "F.Cu") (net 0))
 (segment (start 62.33 74.953257) (end 61.583411 75.699846) (width 0.2) (layer "F.Cu") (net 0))
 (segment (start 70.49 66.935) (end 68.828146 68.596854) (width 0.2) (layer "F.Cu") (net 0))
 (segment (start 52.07 37.02) (end 53.345 35.745) (width 0.2) (layer "F.Cu") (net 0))
 (segment (start 43.345 35.745) (end 41.9 37.19) (width 0.2) (layer "F.Cu") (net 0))
 (segment (start 32.146589 61.303411) (end 30.710154 61.303411) (width 0.2) (layer "F.Cu") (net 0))
 (segment (start 35.284758 37.19) (end 34.892905 37.581853) (width 0.2) (layer "F.Cu") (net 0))
 (segment (start 68.828146 68.596854) (end 68.828146 71.517095) (width 0.2) (layer "F.Cu") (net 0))
 (segment (start 43.345 55.365) (end 40.73 57.98) (width 0.2) (layer "F.Cu") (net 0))
 (segment (start 60.995 40.105) (end 47.61 40.105) (width 0.2) (layer "F.Cu") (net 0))
 (segment (start 73.345 53.065) (end 72.815 53.595) (width 0.2) (layer "F.Cu") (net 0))
 (segment (start 65.99 73.324137) (end 65.38875 73.925387) (width 0.2) (layer "F.Cu") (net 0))
 (segment (start 35.868363 61.725) (end 32.484613 65.10875) (width 0.2) (layer "F.Cu") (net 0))
 (segment (start 38.345 44.405) (end 31.131743 44.405) (width 0.2) (layer "F.Cu") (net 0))
 (segment (start 32.775863 40.73) (end 42.395 40.73) (width 0.2) (layer "F.Cu") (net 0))
 (segment (start 58.345 68.33) (end 53.345 73.33) (width 0.2) (layer "F.Cu") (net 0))
 (segment (start 72.815 53.595) (end 72.815 67.530241) (width 0.2) (layer "F.Cu") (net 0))
 (segment (start 58.345 44.405) (end 58.345 57.17) (width 0.2) (layer "F.Cu") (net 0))
 (segment (start 43.345 71.881637) (end 41.30125 73.925387) (width 0.2) (layer "F.Cu") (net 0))
 (segment (start 68.345 61.725) (end 68.345 65.4) (width 0.2) (layer "F.Cu") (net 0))
 (segment (start 72.815 67.530241) (end 71.797095 68.548146) (width 0.2) (layer "F.Cu") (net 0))
 (segment (start 53.345 73.33) (end 53.345 77.1525) (width 0.2) (layer "F.Cu") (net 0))
 (segment (start 47.653949 61.725) (end 37.861854 71.517095) (width 0.2) (layer "F.Cu") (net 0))
 (segment (start 51.02 53.065) (end 35.536854 68.548146) (width 0.2) (layer "F.Cu") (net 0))
 (segment (start 70.49 58.425) (end 70.49 66.935) (width 0.2) (layer "F.Cu") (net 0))
 (segment (start 40.73 57.98) (end 35.47 57.98) (width 0.2) (layer "F.Cu") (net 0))
 (segment (start 31.131743 44.405) (end 30.710154 44.826589) (width 0.2) (layer "F.Cu") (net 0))
 (segment (start 46.105 37.02) (end 52.07 37.02) (width 0.2) (layer "F.Cu") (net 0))
 (segment (start 63.345 35.745) (end 63.345 37.755) (width 0.2) (layer "F.Cu") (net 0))
 (via blind (at 38.345 44.405) (size 0.25) (drill 0.15) (layers "F.Cu" "B.Cu") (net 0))
 (via blind (at 43.345 70.385) (size 0.25) (drill 0.15) (layers "F.Cu" "B.Cu") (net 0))
 (via blind (at 68.345 44.405) (size 0.25) (drill 0.15) (layers "F.Cu" "B.Cu") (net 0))
 (via blind (at 48.345 61.725) (size 0.25) (drill 0.15) (layers "F.Cu" "B.Cu") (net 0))
 (via blind (at 68.345 61.725) (size 0.25) (drill 0.15) (layers "F.Cu" "B.Cu") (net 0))
 (via blind (at 78.345 44.405) (size 0.25) (drill 0.15) (layers "F.Cu" "B.Cu") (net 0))
 (via blind (at 48.345 44.405) (size 0.25) (drill 0.15) (layers "F.Cu" "B.Cu") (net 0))
 (via blind (at 53.345 70.385) (size 0.25) (drill 0.15) (layers "F.Cu" "B.Cu") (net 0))
 (via blind (at 63.345 70.385) (size 0.25) (drill 0.15) (layers "F.Cu" "B.Cu") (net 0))
 (via blind (at 53.345 35.745) (size 0.25) (drill 0.15) (layers "F.Cu" "B.Cu") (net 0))
 (via blind (at 58.345 44.405) (size 0.25) (drill 0.15) (layers "F.Cu" "B.Cu") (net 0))
 (via blind (at 53.345 53.065) (size 0.25) (drill 0.15) (layers "F.Cu" "B.Cu") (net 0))
 (via blind (at 38.345 61.725) (size 0.25) (drill 0.15) (layers "F.Cu" "B.Cu") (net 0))
 (via blind (at 33.345 53.065) (size 0.25) (drill 0.15) (layers "F.Cu" "B.Cu") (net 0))
 (via blind (at 73.345 53.065) (size 0.25) (drill 0.15) (layers "F.Cu" "B.Cu") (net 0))
 (via blind (at 63.345 35.745) (size 0.25) (drill 0.15) (layers "F.Cu" "B.Cu") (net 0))
 (via blind (at 43.345 53.065) (size 0.25) (drill 0.15) (layers "F.Cu" "B.Cu") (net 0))
 (via blind (at 63.345 53.065) (size 0.25) (drill 0.15) (layers "F.Cu" "B.Cu") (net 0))
 (via blind (at 58.345 61.725) (size 0.25) (drill 0.15) (layers "F.Cu" "B.Cu") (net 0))
 (via blind (at 43.345 35.745) (size 0.25) (drill 0.15) (layers "F.Cu" "B.Cu") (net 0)))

